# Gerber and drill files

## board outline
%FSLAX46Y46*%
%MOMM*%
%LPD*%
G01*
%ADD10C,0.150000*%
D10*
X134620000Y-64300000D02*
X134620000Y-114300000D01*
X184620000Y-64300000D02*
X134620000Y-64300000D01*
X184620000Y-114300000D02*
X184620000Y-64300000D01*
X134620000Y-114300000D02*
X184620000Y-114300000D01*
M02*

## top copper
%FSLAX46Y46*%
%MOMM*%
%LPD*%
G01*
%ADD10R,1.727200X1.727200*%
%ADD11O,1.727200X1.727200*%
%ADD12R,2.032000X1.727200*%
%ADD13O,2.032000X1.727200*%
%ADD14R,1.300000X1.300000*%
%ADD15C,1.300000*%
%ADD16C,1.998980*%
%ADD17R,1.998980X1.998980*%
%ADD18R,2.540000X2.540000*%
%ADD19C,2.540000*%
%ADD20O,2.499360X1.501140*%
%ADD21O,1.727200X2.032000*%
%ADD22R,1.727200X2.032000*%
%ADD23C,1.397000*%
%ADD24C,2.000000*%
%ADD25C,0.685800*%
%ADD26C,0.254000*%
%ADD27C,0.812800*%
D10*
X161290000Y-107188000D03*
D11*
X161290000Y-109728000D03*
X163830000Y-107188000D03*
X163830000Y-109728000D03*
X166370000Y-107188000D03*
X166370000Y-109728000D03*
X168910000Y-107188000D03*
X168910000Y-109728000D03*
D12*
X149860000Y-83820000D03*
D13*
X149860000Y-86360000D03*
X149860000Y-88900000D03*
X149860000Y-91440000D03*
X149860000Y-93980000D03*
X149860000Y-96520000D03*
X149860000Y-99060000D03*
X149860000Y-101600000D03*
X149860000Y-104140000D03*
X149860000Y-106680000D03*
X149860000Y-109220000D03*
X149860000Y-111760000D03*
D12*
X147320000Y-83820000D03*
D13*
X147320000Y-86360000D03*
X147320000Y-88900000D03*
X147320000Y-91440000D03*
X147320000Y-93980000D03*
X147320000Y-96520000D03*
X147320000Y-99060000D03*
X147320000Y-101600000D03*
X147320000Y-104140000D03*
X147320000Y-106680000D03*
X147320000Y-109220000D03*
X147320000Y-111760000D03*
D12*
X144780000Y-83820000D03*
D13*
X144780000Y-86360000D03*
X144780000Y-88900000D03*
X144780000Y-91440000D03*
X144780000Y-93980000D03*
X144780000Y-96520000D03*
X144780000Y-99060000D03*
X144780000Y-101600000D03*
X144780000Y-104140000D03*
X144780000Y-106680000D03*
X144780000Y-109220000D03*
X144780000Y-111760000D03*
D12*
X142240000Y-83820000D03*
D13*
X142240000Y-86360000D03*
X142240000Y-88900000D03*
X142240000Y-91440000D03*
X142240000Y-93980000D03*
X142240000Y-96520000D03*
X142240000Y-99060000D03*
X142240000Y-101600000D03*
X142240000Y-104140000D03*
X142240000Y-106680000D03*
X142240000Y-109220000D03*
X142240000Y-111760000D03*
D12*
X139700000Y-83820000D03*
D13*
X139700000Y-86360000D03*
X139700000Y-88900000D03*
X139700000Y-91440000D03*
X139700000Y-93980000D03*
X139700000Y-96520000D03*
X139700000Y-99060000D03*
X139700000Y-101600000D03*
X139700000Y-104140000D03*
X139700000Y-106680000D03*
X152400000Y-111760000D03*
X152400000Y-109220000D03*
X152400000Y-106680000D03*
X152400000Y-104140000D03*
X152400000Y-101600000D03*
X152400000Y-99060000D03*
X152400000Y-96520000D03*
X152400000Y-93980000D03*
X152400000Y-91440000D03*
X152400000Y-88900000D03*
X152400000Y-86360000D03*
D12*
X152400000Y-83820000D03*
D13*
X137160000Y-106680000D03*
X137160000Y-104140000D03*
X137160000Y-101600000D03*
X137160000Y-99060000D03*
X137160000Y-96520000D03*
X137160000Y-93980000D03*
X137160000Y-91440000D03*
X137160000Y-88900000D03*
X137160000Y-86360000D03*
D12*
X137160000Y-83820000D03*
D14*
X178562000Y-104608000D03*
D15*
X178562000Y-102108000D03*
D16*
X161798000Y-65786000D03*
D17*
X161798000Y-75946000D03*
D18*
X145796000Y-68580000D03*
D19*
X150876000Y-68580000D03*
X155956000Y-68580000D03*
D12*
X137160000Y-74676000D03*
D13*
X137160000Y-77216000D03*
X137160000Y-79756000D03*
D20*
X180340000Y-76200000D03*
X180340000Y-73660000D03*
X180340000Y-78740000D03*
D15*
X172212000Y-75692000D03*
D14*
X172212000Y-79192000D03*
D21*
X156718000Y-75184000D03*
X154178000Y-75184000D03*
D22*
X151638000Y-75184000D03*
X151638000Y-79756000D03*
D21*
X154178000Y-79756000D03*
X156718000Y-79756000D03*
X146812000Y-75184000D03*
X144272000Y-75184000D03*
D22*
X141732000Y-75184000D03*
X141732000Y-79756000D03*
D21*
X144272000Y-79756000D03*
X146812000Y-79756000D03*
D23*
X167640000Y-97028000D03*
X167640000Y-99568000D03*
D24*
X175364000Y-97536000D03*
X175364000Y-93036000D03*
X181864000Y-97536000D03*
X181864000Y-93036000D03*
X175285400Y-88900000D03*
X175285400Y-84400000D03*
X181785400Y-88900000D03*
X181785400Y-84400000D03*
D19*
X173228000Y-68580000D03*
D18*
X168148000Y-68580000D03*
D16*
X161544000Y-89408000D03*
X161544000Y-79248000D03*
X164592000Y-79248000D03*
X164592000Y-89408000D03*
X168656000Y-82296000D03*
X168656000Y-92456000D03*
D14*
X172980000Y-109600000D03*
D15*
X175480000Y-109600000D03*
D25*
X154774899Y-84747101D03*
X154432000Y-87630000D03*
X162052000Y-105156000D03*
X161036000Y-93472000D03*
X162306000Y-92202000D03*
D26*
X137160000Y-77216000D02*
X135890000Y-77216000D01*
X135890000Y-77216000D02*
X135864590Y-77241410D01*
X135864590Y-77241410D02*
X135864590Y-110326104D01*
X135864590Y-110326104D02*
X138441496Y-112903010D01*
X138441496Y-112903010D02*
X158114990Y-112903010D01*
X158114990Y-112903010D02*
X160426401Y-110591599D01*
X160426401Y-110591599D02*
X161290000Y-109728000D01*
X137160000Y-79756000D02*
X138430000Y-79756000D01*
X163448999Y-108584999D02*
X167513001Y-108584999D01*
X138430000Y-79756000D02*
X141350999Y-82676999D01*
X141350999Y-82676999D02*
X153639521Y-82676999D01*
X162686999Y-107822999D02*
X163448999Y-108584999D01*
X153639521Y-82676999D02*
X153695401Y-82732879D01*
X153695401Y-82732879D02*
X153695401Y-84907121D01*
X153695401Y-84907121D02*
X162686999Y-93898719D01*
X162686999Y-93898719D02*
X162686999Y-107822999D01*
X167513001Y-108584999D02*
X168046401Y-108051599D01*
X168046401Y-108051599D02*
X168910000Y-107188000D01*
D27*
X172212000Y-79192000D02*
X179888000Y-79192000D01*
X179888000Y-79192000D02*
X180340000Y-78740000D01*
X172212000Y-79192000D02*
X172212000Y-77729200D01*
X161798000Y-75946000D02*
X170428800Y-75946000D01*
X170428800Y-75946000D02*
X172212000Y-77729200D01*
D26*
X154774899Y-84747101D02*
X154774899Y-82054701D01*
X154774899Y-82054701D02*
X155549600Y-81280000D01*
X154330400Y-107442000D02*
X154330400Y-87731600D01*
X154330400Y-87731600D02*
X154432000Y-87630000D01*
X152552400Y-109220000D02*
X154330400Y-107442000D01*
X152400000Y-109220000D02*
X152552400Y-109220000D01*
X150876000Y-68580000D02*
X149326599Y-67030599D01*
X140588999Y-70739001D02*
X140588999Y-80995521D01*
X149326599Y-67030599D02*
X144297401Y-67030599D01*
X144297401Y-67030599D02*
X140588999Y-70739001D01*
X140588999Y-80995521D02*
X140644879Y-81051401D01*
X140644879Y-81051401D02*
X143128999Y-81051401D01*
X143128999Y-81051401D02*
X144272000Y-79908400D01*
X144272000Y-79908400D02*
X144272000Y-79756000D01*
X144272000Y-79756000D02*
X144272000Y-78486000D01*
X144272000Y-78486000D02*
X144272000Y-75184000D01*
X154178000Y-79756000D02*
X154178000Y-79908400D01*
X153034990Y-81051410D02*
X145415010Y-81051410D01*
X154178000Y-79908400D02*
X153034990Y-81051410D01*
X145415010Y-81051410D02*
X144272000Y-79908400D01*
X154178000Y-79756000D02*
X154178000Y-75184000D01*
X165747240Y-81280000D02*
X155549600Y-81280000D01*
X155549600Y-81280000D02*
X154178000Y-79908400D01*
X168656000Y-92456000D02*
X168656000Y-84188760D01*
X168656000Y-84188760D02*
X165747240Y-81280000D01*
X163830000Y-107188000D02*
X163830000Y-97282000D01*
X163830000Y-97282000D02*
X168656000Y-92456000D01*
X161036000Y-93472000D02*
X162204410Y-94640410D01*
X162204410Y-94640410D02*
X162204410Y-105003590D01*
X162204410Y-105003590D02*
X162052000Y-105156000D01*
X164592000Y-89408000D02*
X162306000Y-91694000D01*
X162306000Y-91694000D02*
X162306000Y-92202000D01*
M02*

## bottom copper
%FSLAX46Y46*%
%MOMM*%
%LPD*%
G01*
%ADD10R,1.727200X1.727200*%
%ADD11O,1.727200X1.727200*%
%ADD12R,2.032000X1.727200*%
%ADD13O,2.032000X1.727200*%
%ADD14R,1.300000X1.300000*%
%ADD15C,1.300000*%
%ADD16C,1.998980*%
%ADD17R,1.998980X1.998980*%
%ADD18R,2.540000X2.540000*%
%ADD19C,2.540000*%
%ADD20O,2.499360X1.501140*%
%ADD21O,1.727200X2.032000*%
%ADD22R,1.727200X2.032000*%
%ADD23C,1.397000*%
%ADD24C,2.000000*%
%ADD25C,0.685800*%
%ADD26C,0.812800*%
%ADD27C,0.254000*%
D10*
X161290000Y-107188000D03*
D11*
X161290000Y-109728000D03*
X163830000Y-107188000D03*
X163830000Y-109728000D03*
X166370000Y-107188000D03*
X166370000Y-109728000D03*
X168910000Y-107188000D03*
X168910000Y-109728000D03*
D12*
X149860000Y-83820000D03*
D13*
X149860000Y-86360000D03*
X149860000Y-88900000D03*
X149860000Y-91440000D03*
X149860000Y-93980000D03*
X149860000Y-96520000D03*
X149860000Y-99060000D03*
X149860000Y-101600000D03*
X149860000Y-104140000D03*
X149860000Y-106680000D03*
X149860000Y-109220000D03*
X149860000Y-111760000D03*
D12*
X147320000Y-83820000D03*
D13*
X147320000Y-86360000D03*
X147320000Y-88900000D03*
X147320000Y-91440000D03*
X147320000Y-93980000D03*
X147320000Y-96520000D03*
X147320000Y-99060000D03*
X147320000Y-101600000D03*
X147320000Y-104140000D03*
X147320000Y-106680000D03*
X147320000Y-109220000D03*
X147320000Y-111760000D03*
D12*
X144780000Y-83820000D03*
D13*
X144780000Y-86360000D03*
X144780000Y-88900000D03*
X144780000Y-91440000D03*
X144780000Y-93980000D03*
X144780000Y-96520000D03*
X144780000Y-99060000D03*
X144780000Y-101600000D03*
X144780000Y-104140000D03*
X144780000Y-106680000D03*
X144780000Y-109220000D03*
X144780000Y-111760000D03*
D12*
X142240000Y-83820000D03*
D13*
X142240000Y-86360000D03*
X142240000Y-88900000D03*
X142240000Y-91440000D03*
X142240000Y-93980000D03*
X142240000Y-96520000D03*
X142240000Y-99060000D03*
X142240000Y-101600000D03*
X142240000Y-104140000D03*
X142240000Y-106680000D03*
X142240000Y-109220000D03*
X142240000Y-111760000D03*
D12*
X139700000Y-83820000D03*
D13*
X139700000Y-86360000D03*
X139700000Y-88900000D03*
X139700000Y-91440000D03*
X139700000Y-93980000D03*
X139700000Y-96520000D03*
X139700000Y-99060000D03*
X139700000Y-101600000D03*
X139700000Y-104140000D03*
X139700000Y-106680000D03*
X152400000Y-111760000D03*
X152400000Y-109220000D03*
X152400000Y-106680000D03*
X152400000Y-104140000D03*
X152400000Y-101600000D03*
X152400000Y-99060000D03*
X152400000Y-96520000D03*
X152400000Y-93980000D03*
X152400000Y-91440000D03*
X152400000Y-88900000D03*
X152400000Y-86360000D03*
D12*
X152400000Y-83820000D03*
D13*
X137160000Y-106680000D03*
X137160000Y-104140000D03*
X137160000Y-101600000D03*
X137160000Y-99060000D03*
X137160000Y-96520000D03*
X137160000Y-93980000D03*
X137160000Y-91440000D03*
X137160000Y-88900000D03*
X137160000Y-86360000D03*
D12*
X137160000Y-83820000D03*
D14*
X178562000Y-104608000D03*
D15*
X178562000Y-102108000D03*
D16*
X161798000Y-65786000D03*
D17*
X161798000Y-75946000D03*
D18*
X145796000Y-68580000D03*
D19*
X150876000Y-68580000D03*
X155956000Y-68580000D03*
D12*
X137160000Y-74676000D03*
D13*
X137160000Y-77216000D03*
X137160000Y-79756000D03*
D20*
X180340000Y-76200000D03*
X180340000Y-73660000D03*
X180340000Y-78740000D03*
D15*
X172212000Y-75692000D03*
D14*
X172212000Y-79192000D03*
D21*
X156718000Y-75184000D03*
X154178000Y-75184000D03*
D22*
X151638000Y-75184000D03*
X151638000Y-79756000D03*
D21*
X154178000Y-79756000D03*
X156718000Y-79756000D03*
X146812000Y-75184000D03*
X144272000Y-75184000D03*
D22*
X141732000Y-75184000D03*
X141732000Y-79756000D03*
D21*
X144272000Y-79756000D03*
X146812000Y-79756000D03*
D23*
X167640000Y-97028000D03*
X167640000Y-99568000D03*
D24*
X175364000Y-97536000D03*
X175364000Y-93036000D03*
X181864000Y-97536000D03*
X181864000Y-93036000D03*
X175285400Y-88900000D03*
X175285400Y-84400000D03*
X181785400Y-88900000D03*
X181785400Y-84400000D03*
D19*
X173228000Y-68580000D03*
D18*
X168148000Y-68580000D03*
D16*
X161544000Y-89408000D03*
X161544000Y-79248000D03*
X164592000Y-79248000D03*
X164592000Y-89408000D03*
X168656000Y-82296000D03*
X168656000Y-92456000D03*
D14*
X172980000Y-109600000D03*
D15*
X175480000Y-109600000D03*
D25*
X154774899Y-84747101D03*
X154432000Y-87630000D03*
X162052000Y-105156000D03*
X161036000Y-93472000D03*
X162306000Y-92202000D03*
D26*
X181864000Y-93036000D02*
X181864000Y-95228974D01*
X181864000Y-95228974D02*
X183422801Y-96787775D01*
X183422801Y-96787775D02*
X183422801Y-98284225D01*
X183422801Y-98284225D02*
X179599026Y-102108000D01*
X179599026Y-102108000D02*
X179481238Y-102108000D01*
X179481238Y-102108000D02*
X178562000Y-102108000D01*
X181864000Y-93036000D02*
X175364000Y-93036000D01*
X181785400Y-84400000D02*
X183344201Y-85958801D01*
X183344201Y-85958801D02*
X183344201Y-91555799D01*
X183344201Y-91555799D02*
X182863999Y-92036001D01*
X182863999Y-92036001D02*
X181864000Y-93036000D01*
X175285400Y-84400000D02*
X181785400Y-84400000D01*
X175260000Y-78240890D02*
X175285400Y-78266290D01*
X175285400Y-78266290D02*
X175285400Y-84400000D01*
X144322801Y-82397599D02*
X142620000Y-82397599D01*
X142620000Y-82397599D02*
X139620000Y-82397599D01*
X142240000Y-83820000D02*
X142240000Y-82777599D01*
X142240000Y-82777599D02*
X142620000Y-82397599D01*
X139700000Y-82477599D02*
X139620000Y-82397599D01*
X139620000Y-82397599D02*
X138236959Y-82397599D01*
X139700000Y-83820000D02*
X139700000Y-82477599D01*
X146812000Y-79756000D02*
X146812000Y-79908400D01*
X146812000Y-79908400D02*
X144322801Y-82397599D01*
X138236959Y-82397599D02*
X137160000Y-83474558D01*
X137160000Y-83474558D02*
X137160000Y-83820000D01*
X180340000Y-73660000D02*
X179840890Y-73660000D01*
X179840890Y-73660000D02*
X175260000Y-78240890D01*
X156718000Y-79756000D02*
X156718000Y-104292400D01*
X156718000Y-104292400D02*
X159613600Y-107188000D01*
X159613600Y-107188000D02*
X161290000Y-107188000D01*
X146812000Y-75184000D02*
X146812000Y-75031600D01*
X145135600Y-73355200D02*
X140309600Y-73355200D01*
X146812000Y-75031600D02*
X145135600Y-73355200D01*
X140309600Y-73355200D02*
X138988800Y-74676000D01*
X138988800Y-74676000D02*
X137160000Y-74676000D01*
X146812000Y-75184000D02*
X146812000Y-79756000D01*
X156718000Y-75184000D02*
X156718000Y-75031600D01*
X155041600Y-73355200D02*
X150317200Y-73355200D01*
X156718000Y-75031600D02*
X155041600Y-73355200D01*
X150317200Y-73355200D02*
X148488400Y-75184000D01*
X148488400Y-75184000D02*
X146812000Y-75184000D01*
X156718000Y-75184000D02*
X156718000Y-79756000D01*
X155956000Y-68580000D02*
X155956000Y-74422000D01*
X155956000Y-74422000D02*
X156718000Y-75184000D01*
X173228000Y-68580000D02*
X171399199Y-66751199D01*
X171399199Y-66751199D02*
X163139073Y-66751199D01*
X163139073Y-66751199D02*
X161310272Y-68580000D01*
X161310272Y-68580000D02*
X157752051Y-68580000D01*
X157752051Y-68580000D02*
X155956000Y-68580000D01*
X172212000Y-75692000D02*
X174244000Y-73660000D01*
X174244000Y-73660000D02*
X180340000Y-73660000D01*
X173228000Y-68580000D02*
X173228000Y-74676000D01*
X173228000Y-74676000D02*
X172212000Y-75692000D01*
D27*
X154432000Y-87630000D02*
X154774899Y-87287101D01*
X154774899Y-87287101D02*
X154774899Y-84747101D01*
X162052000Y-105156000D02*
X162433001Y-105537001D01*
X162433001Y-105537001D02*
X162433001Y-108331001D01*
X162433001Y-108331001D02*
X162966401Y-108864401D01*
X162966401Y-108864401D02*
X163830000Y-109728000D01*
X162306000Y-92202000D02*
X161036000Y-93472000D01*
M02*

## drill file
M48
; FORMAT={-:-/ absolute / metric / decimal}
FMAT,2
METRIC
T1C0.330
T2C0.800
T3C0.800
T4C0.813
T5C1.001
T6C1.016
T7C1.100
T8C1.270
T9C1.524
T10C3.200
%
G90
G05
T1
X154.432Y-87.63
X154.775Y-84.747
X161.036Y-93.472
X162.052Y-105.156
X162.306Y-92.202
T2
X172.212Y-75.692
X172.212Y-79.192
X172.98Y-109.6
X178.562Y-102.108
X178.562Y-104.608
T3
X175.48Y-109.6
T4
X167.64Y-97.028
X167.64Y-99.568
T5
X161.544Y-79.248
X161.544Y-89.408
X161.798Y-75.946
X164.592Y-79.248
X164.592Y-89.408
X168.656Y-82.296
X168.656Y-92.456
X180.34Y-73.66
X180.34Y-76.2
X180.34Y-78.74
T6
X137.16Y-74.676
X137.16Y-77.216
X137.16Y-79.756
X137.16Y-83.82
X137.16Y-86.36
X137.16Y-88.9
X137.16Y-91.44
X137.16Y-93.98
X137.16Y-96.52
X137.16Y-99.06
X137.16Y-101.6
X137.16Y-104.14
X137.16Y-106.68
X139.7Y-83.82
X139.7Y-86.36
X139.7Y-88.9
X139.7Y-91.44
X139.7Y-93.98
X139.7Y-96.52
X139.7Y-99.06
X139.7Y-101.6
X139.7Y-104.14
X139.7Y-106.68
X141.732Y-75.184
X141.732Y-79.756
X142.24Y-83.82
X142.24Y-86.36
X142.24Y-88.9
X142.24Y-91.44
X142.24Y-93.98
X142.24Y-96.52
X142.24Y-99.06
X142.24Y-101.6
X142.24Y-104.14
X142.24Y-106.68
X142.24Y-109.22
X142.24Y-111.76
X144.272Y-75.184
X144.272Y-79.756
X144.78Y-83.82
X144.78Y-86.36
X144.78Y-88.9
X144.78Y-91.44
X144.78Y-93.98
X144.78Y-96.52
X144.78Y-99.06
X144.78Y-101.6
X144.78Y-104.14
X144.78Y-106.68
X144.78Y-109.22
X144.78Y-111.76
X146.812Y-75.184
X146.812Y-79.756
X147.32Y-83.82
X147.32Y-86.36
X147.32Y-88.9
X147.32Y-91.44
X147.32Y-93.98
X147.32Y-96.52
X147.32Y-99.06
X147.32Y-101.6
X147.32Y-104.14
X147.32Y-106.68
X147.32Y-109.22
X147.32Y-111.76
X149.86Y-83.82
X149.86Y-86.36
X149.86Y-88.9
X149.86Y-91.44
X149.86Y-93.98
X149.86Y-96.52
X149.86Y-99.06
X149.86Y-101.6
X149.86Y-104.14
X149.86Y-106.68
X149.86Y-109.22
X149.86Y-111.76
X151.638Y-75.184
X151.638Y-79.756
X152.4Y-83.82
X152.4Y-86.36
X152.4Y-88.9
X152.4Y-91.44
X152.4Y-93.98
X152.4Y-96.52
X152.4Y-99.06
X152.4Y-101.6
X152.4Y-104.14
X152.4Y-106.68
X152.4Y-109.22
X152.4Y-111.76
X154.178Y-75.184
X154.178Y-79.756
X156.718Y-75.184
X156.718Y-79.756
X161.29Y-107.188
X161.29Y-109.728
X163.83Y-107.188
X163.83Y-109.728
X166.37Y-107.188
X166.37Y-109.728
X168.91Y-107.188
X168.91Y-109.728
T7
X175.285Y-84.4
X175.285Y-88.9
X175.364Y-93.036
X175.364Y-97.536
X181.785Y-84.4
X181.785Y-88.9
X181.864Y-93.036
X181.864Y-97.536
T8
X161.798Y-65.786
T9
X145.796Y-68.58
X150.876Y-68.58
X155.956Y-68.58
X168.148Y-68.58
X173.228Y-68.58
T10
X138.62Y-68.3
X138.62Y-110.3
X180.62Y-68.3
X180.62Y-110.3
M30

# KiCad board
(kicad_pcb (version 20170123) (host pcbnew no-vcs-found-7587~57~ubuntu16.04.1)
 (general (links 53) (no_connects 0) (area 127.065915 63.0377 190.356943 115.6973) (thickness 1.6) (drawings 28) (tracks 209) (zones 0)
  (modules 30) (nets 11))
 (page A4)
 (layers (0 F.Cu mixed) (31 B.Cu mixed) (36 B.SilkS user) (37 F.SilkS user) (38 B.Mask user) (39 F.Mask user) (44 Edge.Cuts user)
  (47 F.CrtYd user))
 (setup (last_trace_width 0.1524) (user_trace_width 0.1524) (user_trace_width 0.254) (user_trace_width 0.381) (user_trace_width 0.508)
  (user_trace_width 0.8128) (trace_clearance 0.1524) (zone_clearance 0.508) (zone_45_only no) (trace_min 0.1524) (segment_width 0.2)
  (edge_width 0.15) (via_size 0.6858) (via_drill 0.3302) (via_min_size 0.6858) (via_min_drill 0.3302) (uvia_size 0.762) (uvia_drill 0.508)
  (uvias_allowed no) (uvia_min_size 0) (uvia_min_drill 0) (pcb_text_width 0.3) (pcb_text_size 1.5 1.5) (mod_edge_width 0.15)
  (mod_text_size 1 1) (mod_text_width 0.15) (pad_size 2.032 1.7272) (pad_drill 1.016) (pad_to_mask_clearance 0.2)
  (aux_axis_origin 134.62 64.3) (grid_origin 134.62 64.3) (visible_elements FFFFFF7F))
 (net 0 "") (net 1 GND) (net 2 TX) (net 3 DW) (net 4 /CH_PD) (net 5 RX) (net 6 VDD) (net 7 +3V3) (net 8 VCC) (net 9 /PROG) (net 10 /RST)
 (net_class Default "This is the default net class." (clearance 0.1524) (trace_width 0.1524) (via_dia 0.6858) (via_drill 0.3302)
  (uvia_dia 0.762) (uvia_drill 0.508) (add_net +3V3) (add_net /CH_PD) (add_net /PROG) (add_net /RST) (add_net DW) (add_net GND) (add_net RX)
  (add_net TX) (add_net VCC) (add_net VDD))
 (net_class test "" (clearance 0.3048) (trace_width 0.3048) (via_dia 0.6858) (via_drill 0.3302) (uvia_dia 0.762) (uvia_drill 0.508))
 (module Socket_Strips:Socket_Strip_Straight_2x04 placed (layer F.Cu) (at 161.29 107.188)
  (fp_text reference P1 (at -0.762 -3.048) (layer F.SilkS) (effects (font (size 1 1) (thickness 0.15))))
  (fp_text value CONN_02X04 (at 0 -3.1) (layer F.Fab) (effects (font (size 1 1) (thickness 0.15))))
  (pad 1 thru_hole rect (at 0 0) (size 1.7272 1.7272) (drill 1.016) (layers *.Cu *.Mask) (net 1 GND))
  (pad 2 thru_hole oval (at 0 2.54) (size 1.7272 1.7272) (drill 1.016) (layers *.Cu *.Mask) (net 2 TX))
  (pad 3 thru_hole oval (at 2.54 0) (size 1.7272 1.7272) (drill 1.016) (layers *.Cu *.Mask) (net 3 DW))
  (pad 4 thru_hole oval (at 2.54 2.54) (size 1.7272 1.7272) (drill 1.016) (layers *.Cu *.Mask) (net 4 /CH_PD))
  (pad 5 thru_hole oval (at 5.08 0) (size 1.7272 1.7272) (drill 1.016) (layers *.Cu *.Mask))
  (pad 6 thru_hole oval (at 5.08 2.54) (size 1.7272 1.7272) (drill 1.016) (layers *.Cu *.Mask))
  (pad 7 thru_hole oval (at 7.62 0) (size 1.7272 1.7272) (drill 1.016) (layers *.Cu *.Mask) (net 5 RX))
  (pad 8 thru_hole oval (at 7.62 2.54) (size 1.7272 1.7272) (drill 1.016) (layers *.Cu *.Mask)))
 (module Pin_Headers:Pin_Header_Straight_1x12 (layer F.Cu) (at 149.86 83.82)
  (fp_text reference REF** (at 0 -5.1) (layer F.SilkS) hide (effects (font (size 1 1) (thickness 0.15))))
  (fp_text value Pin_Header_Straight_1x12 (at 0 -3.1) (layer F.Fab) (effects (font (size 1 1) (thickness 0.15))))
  (pad 1 thru_hole rect (at 0 0) (size 2.032 1.7272) (drill 1.016) (layers *.Cu *.Mask))
  (pad 2 thru_hole oval (at 0 2.54) (size 2.032 1.7272) (drill 1.016) (layers *.Cu *.Mask))
  (pad 3 thru_hole oval (at 0 5.08) (size 2.032 1.7272) (drill 1.016) (layers *.Cu *.Mask))
  (pad 4 thru_hole oval (at 0 7.62) (size 2.032 1.7272) (drill 1.016) (layers *.Cu *.Mask))
  (pad 5 thru_hole oval (at 0 10.16) (size 2.032 1.7272) (drill 1.016) (layers *.Cu *.Mask))
  (pad 6 thru_hole oval (at 0 12.7) (size 2.032 1.7272) (drill 1.016) (layers *.Cu *.Mask))
  (pad 7 thru_hole oval (at 0 15.24) (size 2.032 1.7272) (drill 1.016) (layers *.Cu *.Mask))
  (pad 8 thru_hole oval (at 0 17.78) (size 2.032 1.7272) (drill 1.016) (layers *.Cu *.Mask))
  (pad 9 thru_hole oval (at 0 20.32) (size 2.032 1.7272) (drill 1.016) (layers *.Cu *.Mask))
  (pad 10 thru_hole oval (at 0 22.86) (size 2.032 1.7272) (drill 1.016) (layers *.Cu *.Mask))
  (pad 11 thru_hole oval (at 0 25.4) (size 2.032 1.7272) (drill 1.016) (layers *.Cu *.Mask))
  (pad 12 thru_hole oval (at 0 27.94) (size 2.032 1.7272) (drill 1.016) (layers *.Cu *.Mask)))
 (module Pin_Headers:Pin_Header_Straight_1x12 (layer F.Cu) (at 147.32 83.82)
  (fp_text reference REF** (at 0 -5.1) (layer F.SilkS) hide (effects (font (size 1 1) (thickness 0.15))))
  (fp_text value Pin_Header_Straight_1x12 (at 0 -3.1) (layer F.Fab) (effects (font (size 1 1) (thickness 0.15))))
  (pad 1 thru_hole rect (at 0 0) (size 2.032 1.7272) (drill 1.016) (layers *.Cu *.Mask))
  (pad 2 thru_hole oval (at 0 2.54) (size 2.032 1.7272) (drill 1.016) (layers *.Cu *.Mask))
  (pad 3 thru_hole oval (at 0 5.08) (size 2.032 1.7272) (drill 1.016) (layers *.Cu *.Mask))
  (pad 4 thru_hole oval (at 0 7.62) (size 2.032 1.7272) (drill 1.016) (layers *.Cu *.Mask))
  (pad 5 thru_hole oval (at 0 10.16) (size 2.032 1.7272) (drill 1.016) (layers *.Cu *.Mask))
  (pad 6 thru_hole oval (at 0 12.7) (size 2.032 1.7272) (drill 1.016) (layers *.Cu *.Mask))
  (pad 7 thru_hole oval (at 0 15.24) (size 2.032 1.7272) (drill 1.016) (layers *.Cu *.Mask))
  (pad 8 thru_hole oval (at 0 17.78) (size 2.032 1.7272) (drill 1.016) (layers *.Cu *.Mask))
  (pad 9 thru_hole oval (at 0 20.32) (size 2.032 1.7272) (drill 1.016) (layers *.Cu *.Mask))
  (pad 10 thru_hole oval (at 0 22.86) (size 2.032 1.7272) (drill 1.016) (layers *.Cu *.Mask))
  (pad 11 thru_hole oval (at 0 25.4) (size 2.032 1.7272) (drill 1.016) (layers *.Cu *.Mask))
  (pad 12 thru_hole oval (at 0 27.94) (size 2.032 1.7272) (drill 1.016) (layers *.Cu *.Mask)))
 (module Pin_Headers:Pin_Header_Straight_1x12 (layer F.Cu) (at 144.78 83.82)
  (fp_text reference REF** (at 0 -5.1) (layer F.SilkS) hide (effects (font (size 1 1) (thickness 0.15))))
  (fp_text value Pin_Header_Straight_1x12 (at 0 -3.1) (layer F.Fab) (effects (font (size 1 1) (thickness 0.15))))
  (pad 1 thru_hole rect (at 0 0) (size 2.032 1.7272) (drill 1.016) (layers *.Cu *.Mask))
  (pad 2 thru_hole oval (at 0 2.54) (size 2.032 1.7272) (drill 1.016) (layers *.Cu *.Mask))
  (pad 3 thru_hole oval (at 0 5.08) (size 2.032 1.7272) (drill 1.016) (layers *.Cu *.Mask))
  (pad 4 thru_hole oval (at 0 7.62) (size 2.032 1.7272) (drill 1.016) (layers *.Cu *.Mask))
  (pad 5 thru_hole oval (at 0 10.16) (size 2.032 1.7272) (drill 1.016) (layers *.Cu *.Mask))
  (pad 6 thru_hole oval (at 0 12.7) (size 2.032 1.7272) (drill 1.016) (layers *.Cu *.Mask))
  (pad 7 thru_hole oval (at 0 15.24) (size 2.032 1.7272) (drill 1.016) (layers *.Cu *.Mask))
  (pad 8 thru_hole oval (at 0 17.78) (size 2.032 1.7272) (drill 1.016) (layers *.Cu *.Mask))
  (pad 9 thru_hole oval (at 0 20.32) (size 2.032 1.7272) (drill 1.016) (layers *.Cu *.Mask))
  (pad 10 thru_hole oval (at 0 22.86) (size 2.032 1.7272) (drill 1.016) (layers *.Cu *.Mask))
  (pad 11 thru_hole oval (at 0 25.4) (size 2.032 1.7272) (drill 1.016) (layers *.Cu *.Mask))
  (pad 12 thru_hole oval (at 0 27.94) (size 2.032 1.7272) (drill 1.016) (layers *.Cu *.Mask)))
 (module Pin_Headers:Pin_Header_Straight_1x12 (layer F.Cu) (at 142.24 83.82)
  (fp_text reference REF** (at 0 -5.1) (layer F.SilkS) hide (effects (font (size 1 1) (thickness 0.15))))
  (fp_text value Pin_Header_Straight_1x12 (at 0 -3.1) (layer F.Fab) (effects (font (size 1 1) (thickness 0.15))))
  (pad 1 thru_hole rect (at 0 0) (size 2.032 1.7272) (drill 1.016) (layers *.Cu *.Mask) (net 1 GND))
  (pad 2 thru_hole oval (at 0 2.54) (size 2.032 1.7272) (drill 1.016) (layers *.Cu *.Mask))
  (pad 3 thru_hole oval (at 0 5.08) (size 2.032 1.7272) (drill 1.016) (layers *.Cu *.Mask))
  (pad 4 thru_hole oval (at 0 7.62) (size 2.032 1.7272) (drill 1.016) (layers *.Cu *.Mask))
  (pad 5 thru_hole oval (at 0 10.16) (size 2.032 1.7272) (drill 1.016) (layers *.Cu *.Mask))
  (pad 6 thru_hole oval (at 0 12.7) (size 2.032 1.7272) (drill 1.016) (layers *.Cu *.Mask))
  (pad 7 thru_hole oval (at 0 15.24) (size 2.032 1.7272) (drill 1.016) (layers *.Cu *.Mask))
  (pad 8 thru_hole oval (at 0 17.78) (size 2.032 1.7272) (drill 1.016) (layers *.Cu *.Mask))
  (pad 9 thru_hole oval (at 0 20.32) (size 2.032 1.7272) (drill 1.016) (layers *.Cu *.Mask))
  (pad 10 thru_hole oval (at 0 22.86) (size 2.032 1.7272) (drill 1.016) (layers *.Cu *.Mask))
  (pad 11 thru_hole oval (at 0 25.4) (size 2.032 1.7272) (drill 1.016) (layers *.Cu *.Mask))
  (pad 12 thru_hole oval (at 0 27.94) (size 2.032 1.7272) (drill 1.016) (layers *.Cu *.Mask)))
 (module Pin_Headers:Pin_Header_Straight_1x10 (layer F.Cu) (at 139.7 83.82)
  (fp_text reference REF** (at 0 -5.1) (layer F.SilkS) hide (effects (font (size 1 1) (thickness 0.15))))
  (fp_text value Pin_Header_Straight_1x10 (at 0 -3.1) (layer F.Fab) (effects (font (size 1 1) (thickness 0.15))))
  (pad 1 thru_hole rect (at 0 0) (size 2.032 1.7272) (drill 1.016) (layers *.Cu *.Mask) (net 1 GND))
  (pad 2 thru_hole oval (at 0 2.54) (size 2.032 1.7272) (drill 1.016) (layers *.Cu *.Mask))
  (pad 3 thru_hole oval (at 0 5.08) (size 2.032 1.7272) (drill 1.016) (layers *.Cu *.Mask))
  (pad 4 thru_hole oval (at 0 7.62) (size 2.032 1.7272) (drill 1.016) (layers *.Cu *.Mask))
  (pad 5 thru_hole oval (at 0 10.16) (size 2.032 1.7272) (drill 1.016) (layers *.Cu *.Mask))
  (pad 6 thru_hole oval (at 0 12.7) (size 2.032 1.7272) (drill 1.016) (layers *.Cu *.Mask))
  (pad 7 thru_hole oval (at 0 15.24) (size 2.032 1.7272) (drill 1.016) (layers *.Cu *.Mask))
  (pad 8 thru_hole oval (at 0 17.78) (size 2.032 1.7272) (drill 1.016) (layers *.Cu *.Mask))
  (pad 9 thru_hole oval (at 0 20.32) (size 2.032 1.7272) (drill 1.016) (layers *.Cu *.Mask))
  (pad 10 thru_hole oval (at 0 22.86) (size 2.032 1.7272) (drill 1.016) (layers *.Cu *.Mask)))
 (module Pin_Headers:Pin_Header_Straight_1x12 (layer F.Cu) (at 152.4 83.82)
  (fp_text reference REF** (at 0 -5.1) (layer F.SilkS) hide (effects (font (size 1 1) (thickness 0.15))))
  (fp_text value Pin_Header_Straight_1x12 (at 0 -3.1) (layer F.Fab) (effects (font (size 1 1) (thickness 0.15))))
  (pad 12 thru_hole oval (at 0 27.94) (size 2.032 1.7272) (drill 1.016) (layers *.Cu *.Mask))
  (pad 11 thru_hole oval (at 0 25.4) (size 2.032 1.7272) (drill 1.016) (layers *.Cu *.Mask) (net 3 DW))
  (pad 10 thru_hole oval (at 0 22.86) (size 2.032 1.7272) (drill 1.016) (layers *.Cu *.Mask))
  (pad 9 thru_hole oval (at 0 20.32) (size 2.032 1.7272) (drill 1.016) (layers *.Cu *.Mask))
  (pad 8 thru_hole oval (at 0 17.78) (size 2.032 1.7272) (drill 1.016) (layers *.Cu *.Mask))
  (pad 7 thru_hole oval (at 0 15.24) (size 2.032 1.7272) (drill 1.016) (layers *.Cu *.Mask))
  (pad 6 thru_hole oval (at 0 12.7) (size 2.032 1.7272) (drill 1.016) (layers *.Cu *.Mask))
  (pad 5 thru_hole oval (at 0 10.16) (size 2.032 1.7272) (drill 1.016) (layers *.Cu *.Mask))
  (pad 4 thru_hole oval (at 0 7.62) (size 2.032 1.7272) (drill 1.016) (layers *.Cu *.Mask))
  (pad 3 thru_hole oval (at 0 5.08) (size 2.032 1.7272) (drill 1.016) (layers *.Cu *.Mask))
  (pad 2 thru_hole oval (at 0 2.54) (size 2.032 1.7272) (drill 1.016) (layers *.Cu *.Mask))
  (pad 1 thru_hole rect (at 0 0) (size 2.032 1.7272) (drill 1.016) (layers *.Cu *.Mask)))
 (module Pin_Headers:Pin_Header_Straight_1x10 (layer F.Cu) (at 137.16 83.82)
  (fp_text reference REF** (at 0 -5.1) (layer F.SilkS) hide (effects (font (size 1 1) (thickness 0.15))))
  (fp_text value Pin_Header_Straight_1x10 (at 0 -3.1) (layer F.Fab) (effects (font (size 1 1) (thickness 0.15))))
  (pad 10 thru_hole oval (at 0 22.86) (size 2.032 1.7272) (drill 1.016) (layers *.Cu *.Mask))
  (pad 9 thru_hole oval (at 0 20.32) (size 2.032 1.7272) (drill 1.016) (layers *.Cu *.Mask))
  (pad 8 thru_hole oval (at 0 17.78) (size 2.032 1.7272) (drill 1.016) (layers *.Cu *.Mask))
  (pad 7 thru_hole oval (at 0 15.24) (size 2.032 1.7272) (drill 1.016) (layers *.Cu *.Mask))
  (pad 6 thru_hole oval (at 0 12.7) (size 2.032 1.7272) (drill 1.016) (layers *.Cu *.Mask))
  (pad 5 thru_hole oval (at 0 10.16) (size 2.032 1.7272) (drill 1.016) (layers *.Cu *.Mask))
  (pad 4 thru_hole oval (at 0 7.62) (size 2.032 1.7272) (drill 1.016) (layers *.Cu *.Mask))
  (pad 3 thru_hole oval (at 0 5.08) (size 2.032 1.7272) (drill 1.016) (layers *.Cu *.Mask))
  (pad 2 thru_hole oval (at 0 2.54) (size 2.032 1.7272) (drill 1.016) (layers *.Cu *.Mask))
  (pad 1 thru_hole rect (at 0 0) (size 2.032 1.7272) (drill 1.016) (layers *.Cu *.Mask) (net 1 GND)))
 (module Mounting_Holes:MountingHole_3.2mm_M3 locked (layer F.Cu) (at 180.62 68.3)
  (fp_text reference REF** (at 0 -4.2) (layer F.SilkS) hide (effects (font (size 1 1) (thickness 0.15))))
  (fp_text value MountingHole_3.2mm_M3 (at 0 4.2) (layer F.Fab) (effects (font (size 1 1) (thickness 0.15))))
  (pad 1 np_thru_hole circle (at 0 0) (size 3.2 3.2) (drill 3.2) (layers *.Cu *.Mask)))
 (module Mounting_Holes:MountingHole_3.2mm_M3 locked (layer F.Cu) (at 138.62 68.3)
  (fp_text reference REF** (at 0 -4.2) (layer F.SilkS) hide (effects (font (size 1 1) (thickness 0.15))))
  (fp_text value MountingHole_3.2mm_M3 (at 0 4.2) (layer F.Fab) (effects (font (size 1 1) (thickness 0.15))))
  (pad 1 np_thru_hole circle (at 0 0) (size 3.2 3.2) (drill 3.2) (layers *.Cu *.Mask)))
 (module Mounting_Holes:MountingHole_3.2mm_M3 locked (layer F.Cu) (at 138.62 110.3)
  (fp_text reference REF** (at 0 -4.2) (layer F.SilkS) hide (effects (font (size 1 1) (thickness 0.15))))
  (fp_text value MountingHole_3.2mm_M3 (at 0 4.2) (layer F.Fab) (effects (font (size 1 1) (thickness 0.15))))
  (pad 1 np_thru_hole circle (at 0 0) (size 3.2 3.2) (drill 3.2) (layers *.Cu *.Mask)))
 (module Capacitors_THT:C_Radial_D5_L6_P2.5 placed (layer F.Cu) (at 178.562 104.608 90)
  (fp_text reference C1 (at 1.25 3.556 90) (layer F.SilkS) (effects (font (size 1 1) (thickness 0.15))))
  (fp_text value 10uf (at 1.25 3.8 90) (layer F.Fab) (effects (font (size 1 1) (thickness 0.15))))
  (pad 1 thru_hole rect (at 0 0 90) (size 1.3 1.3) (drill 0.8) (layers *.Cu *.Mask))
  (pad 2 thru_hole circle (at 2.5 0 90) (size 1.3 1.3) (drill 0.8) (layers *.Cu *.Mask) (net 1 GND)))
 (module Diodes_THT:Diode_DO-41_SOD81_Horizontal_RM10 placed (layer F.Cu) (at 161.80054 75.946 90)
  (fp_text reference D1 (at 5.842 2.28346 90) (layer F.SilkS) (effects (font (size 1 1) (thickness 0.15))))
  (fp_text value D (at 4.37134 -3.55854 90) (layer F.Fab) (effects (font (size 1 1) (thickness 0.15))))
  (pad 2 thru_hole circle (at 10.16 -0.00254 270) (size 1.99898 1.99898) (drill 1.27) (layers *.Cu *.Mask))
  (pad 1 thru_hole rect (at 0 -0.00254 270) (size 1.99898 1.99898) (drill 1.00076) (layers *.Cu *.Mask) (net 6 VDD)))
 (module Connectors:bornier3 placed (layer F.Cu) (at 150.876 68.58)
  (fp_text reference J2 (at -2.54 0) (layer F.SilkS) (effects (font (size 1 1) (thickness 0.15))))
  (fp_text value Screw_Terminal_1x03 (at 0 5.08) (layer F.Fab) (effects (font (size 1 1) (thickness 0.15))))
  (pad 1 thru_hole rect (at -5.08 0) (size 2.54 2.54) (drill 1.524) (layers *.Cu *.Mask))
  (pad 2 thru_hole circle (at 0 0) (size 2.54 2.54) (drill 1.524) (layers *.Cu *.Mask) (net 3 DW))
  (pad 3 thru_hole circle (at 5.08 0) (size 2.54 2.54) (drill 1.524) (layers *.Cu *.Mask) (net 1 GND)))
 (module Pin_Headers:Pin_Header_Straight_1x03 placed (layer F.Cu) (at 137.16 74.676)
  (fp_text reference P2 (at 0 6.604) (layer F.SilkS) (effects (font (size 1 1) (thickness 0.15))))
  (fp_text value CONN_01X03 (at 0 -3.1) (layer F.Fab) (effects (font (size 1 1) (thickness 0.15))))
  (pad 1 thru_hole rect (at 0 0) (size 2.032 1.7272) (drill 1.016) (layers *.Cu *.Mask) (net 1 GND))
  (pad 2 thru_hole oval (at 0 2.54) (size 2.032 1.7272) (drill 1.016) (layers *.Cu *.Mask) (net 2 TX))
  (pad 3 thru_hole oval (at 0 5.08) (size 2.032 1.7272) (drill 1.016) (layers *.Cu *.Mask) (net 5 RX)))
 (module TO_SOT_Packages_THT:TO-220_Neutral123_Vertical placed (layer F.Cu) (at 180.34 76.2 270)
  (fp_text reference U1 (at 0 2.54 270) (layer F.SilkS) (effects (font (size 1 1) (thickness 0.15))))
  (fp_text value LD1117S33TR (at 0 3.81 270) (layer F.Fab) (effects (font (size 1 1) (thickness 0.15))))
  (pad 2 thru_hole oval (at 0 0) (size 2.49936 1.50114) (drill 1.00076) (layers *.Cu *.Mask))
  (pad 1 thru_hole oval (at -2.54 0) (size 2.49936 1.50114) (drill 1.00076) (layers *.Cu *.Mask) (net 1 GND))
  (pad 3 thru_hole oval (at 2.54 0) (size 2.49936 1.50114) (drill 1.00076) (layers *.Cu *.Mask) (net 6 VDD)))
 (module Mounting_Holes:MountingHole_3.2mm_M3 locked (layer F.Cu) (at 180.62 110.3)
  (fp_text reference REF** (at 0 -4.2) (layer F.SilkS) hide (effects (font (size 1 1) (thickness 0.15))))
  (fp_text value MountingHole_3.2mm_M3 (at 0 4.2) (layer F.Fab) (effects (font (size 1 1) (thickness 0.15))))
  (pad 1 np_thru_hole circle (at 0 0) (size 3.2 3.2) (drill 3.2) (layers *.Cu *.Mask)))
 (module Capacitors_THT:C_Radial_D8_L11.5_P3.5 (layer F.Cu) (at 172.212 79.192 90)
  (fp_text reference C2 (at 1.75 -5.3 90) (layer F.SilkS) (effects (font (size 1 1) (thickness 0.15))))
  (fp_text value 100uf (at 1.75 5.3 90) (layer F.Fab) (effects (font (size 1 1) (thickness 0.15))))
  (pad 2 thru_hole circle (at 3.5 0 90) (size 1.3 1.3) (drill 0.8) (layers *.Cu *.Mask) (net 1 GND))
  (pad 1 thru_hole rect (at 0 0 90) (size 1.3 1.3) (drill 0.8) (layers *.Cu *.Mask) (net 6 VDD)))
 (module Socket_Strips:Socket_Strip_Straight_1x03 (layer F.Cu) (at 151.638 75.184)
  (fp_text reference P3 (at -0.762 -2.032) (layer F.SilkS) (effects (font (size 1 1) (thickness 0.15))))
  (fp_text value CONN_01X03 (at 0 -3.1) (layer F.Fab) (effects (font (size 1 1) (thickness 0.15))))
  (pad 3 thru_hole oval (at 5.08 0) (size 1.7272 2.032) (drill 1.016) (layers *.Cu *.Mask) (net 1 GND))
  (pad 2 thru_hole oval (at 2.54 0) (size 1.7272 2.032) (drill 1.016) (layers *.Cu *.Mask) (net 3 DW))
  (pad 1 thru_hole rect (at 0 0) (size 1.7272 2.032) (drill 1.016) (layers *.Cu *.Mask)))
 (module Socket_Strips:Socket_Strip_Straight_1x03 (layer F.Cu) (at 151.638 79.756)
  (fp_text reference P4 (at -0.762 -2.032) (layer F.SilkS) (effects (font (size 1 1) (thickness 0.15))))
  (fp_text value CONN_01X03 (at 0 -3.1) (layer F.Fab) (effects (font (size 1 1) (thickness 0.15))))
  (pad 1 thru_hole rect (at 0 0) (size 1.7272 2.032) (drill 1.016) (layers *.Cu *.Mask))
  (pad 2 thru_hole oval (at 2.54 0) (size 1.7272 2.032) (drill 1.016) (layers *.Cu *.Mask) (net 3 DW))
  (pad 3 thru_hole oval (at 5.08 0) (size 1.7272 2.032) (drill 1.016) (layers *.Cu *.Mask) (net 1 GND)))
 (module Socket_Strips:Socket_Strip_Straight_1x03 (layer F.Cu) (at 141.732 75.184)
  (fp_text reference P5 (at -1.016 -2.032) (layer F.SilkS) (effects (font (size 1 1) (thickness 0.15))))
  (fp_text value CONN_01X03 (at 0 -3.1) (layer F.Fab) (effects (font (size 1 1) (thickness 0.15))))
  (pad 3 thru_hole oval (at 5.08 0) (size 1.7272 2.032) (drill 1.016) (layers *.Cu *.Mask) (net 1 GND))
  (pad 2 thru_hole oval (at 2.54 0) (size 1.7272 2.032) (drill 1.016) (layers *.Cu *.Mask) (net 3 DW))
  (pad 1 thru_hole rect (at 0 0) (size 1.7272 2.032) (drill 1.016) (layers *.Cu *.Mask)))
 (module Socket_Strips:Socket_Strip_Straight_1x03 (layer F.Cu) (at 141.732 79.756)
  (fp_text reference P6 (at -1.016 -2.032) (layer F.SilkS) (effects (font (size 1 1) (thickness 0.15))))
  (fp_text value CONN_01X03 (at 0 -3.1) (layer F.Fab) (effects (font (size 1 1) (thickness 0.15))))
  (pad 1 thru_hole rect (at 0 0) (size 1.7272 2.032) (drill 1.016) (layers *.Cu *.Mask))
  (pad 2 thru_hole oval (at 2.54 0) (size 1.7272 2.032) (drill 1.016) (layers *.Cu *.Mask) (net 3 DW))
  (pad 3 thru_hole oval (at 5.08 0) (size 1.7272 2.032) (drill 1.016) (layers *.Cu *.Mask) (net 1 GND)))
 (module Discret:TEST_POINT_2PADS (layer F.Cu) (at 167.64 98.298 270)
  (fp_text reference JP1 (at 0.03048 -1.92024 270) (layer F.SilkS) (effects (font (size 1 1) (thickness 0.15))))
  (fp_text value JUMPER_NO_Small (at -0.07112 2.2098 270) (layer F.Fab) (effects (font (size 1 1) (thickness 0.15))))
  (pad 1 thru_hole circle (at -1.27 0 270) (size 1.397 1.397) (drill 0.8128) (layers *.Cu *.Mask F.SilkS))
  (pad 2 thru_hole circle (at 1.27 0 270) (size 1.397 1.397) (drill 0.8128) (layers *.Cu *.Mask F.SilkS)))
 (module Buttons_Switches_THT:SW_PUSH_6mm (layer F.Cu) (at 181.864 97.536 180)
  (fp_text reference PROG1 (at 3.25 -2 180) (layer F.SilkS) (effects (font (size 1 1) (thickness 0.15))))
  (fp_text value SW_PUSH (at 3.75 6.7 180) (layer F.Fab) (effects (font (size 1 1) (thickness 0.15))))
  (pad 1 thru_hole circle (at 6.5 0 270) (size 2 2) (drill 1.1) (layers *.Cu *.Mask))
  (pad 2 thru_hole circle (at 6.5 4.5 270) (size 2 2) (drill 1.1) (layers *.Cu *.Mask) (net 1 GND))
  (pad 1 thru_hole circle (at 0 0 270) (size 2 2) (drill 1.1) (layers *.Cu *.Mask))
  (pad 2 thru_hole circle (at 0 4.5 270) (size 2 2) (drill 1.1) (layers *.Cu *.Mask) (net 1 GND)))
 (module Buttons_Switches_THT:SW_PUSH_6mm (layer F.Cu) (at 175.2854 84.4)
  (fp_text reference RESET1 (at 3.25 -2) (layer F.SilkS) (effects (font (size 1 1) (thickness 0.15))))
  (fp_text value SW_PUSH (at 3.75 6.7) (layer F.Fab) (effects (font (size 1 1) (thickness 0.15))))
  (pad 2 thru_hole circle (at 0 4.5 90) (size 2 2) (drill 1.1) (layers *.Cu *.Mask))
  (pad 1 thru_hole circle (at 0 0 90) (size 2 2) (drill 1.1) (layers *.Cu *.Mask) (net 1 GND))
  (pad 2 thru_hole circle (at 6.5 4.5 90) (size 2 2) (drill 1.1) (layers *.Cu *.Mask))
  (pad 1 thru_hole circle (at 6.5 0 90) (size 2 2) (drill 1.1) (layers *.Cu *.Mask) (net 1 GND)))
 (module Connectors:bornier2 (layer F.Cu) (at 170.688 68.58)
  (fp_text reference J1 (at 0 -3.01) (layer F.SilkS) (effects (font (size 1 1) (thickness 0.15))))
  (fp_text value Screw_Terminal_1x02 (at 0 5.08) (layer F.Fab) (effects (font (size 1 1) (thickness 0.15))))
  (pad 2 thru_hole circle (at 2.54 0) (size 2.54 2.54) (drill 1.524) (layers *.Cu *.Mask) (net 1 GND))
  (pad 1 thru_hole rect (at -2.54 0) (size 2.54 2.54) (drill 1.524) (layers *.Cu *.Mask)))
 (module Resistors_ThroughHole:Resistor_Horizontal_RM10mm (layer F.Cu) (at 161.544 89.408 90)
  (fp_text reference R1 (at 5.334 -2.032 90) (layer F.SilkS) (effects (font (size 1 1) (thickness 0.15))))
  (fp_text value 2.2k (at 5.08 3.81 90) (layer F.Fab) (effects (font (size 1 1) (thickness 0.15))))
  (pad 1 thru_hole circle (at 0 0 90) (size 1.99898 1.99898) (drill 1.00076) (layers *.Cu *.SilkS *.Mask))
  (pad 2 thru_hole circle (at 10.16 0 90) (size 1.99898 1.99898) (drill 1.00076) (layers *.Cu *.SilkS *.Mask)))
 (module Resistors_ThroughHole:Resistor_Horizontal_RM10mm (layer F.Cu) (at 164.592 89.408 90)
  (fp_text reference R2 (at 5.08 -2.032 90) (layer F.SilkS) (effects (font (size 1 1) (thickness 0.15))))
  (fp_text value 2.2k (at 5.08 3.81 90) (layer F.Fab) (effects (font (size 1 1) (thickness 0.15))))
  (pad 2 thru_hole circle (at 10.16 0 90) (size 1.99898 1.99898) (drill 1.00076) (layers *.Cu *.SilkS *.Mask))
  (pad 1 thru_hole circle (at 0 0 90) (size 1.99898 1.99898) (drill 1.00076) (layers *.Cu *.SilkS *.Mask) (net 4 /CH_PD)))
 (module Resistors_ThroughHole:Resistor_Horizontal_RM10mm (layer F.Cu) (at 168.656 82.296 270)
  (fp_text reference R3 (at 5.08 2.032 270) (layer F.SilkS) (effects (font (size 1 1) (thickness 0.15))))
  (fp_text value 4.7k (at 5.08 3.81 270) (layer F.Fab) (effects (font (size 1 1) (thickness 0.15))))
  (pad 1 thru_hole circle (at 0 0 270) (size 1.99898 1.99898) (drill 1.00076) (layers *.Cu *.SilkS *.Mask))
  (pad 2 thru_hole circle (at 10.16 0 270) (size 1.99898 1.99898) (drill 1.00076) (layers *.Cu *.SilkS *.Mask) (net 3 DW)))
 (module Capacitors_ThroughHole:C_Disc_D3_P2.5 (layer F.Cu) (at 172.98 109.6)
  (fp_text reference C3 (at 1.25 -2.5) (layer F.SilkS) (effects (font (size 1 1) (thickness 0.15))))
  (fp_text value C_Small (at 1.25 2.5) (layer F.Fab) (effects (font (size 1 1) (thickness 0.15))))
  (pad 1 thru_hole rect (at 0 0) (size 1.3 1.3) (drill 0.8) (layers *.Cu *.Mask F.SilkS))
  (pad 2 thru_hole circle (at 2.5 0) (size 1.3 1.3) (drill 0.8001) (layers *.Cu *.Mask F.SilkS)))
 (gr_line (start 134.62 64.3) (end 134.62 114.3) (angle 90) (layer Edge.Cuts) (width 0.15))
 (gr_line (start 184.62 64.3) (end 134.62 64.3) (angle 90) (layer Edge.Cuts) (width 0.15))
 (gr_line (start 184.62 114.3) (end 184.62 64.3) (angle 90) (layer Edge.Cuts) (width 0.15))
 (gr_line (start 134.62 114.3) (end 184.62 114.3) (angle 90) (layer Edge.Cuts) (width 0.15))
 (segment (start 181.864 93.036) (end 181.864 95.228974) (width 0.8128) (layer B.Cu) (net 1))
 (segment (start 181.864 95.228974) (end 183.422801 96.787775) (width 0.8128) (layer B.Cu) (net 1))
 (segment (start 183.422801 96.787775) (end 183.422801 98.284225) (width 0.8128) (layer B.Cu) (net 1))
 (segment (start 183.422801 98.284225) (end 179.599026 102.108) (width 0.8128) (layer B.Cu) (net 1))
 (segment (start 179.599026 102.108) (end 179.481238 102.108) (width 0.8128) (layer B.Cu) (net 1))
 (segment (start 179.481238 102.108) (end 178.562 102.108) (width 0.8128) (layer B.Cu) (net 1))
 (segment (start 181.864 93.036) (end 175.364 93.036) (width 0.8128) (layer B.Cu) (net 1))
 (segment (start 181.7854 84.4) (end 183.344201 85.958801) (width 0.8128) (layer B.Cu) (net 1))
 (segment (start 183.344201 85.958801) (end 183.344201 91.555799) (width 0.8128) (layer B.Cu) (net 1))
 (segment (start 183.344201 91.555799) (end 182.863999 92.036001) (width 0.8128) (layer B.Cu) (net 1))
 (segment (start 182.863999 92.036001) (end 181.864 93.036) (width 0.8128) (layer B.Cu) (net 1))
 (segment (start 175.2854 84.4) (end 181.7854 84.4) (width 0.8128) (layer B.Cu) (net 1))
 (segment (start 175.26 78.24089) (end 175.2854 78.26629) (width 0.8128) (layer B.Cu) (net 1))
 (segment (start 175.2854 78.26629) (end 175.2854 84.4) (width 0.8128) (layer B.Cu) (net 1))
 (segment (start 144.322801 82.397599) (end 142.62 82.397599) (width 0.8128) (layer B.Cu) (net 1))
 (segment (start 142.62 82.397599) (end 139.62 82.397599) (width 0.8128) (layer B.Cu) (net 1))
 (segment (start 142.24 83.82) (end 142.24 82.777599) (width 0.8128) (layer B.Cu) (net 1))
 (segment (start 142.24 82.777599) (end 142.62 82.397599) (width 0.8128) (layer B.Cu) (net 1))
 (segment (start 139.7 82.477599) (end 139.62 82.397599) (width 0.8128) (layer B.Cu) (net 1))
 (segment (start 139.62 82.397599) (end 138.236959 82.397599) (width 0.8128) (layer B.Cu) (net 1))
 (segment (start 139.7 83.82) (end 139.7 82.477599) (width 0.8128) (layer B.Cu) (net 1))
 (segment (start 146.812 79.756) (end 146.812 79.9084) (width 0.8128) (layer B.Cu) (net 1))
 (segment (start 146.812 79.9084) (end 144.322801 82.397599) (width 0.8128) (layer B.Cu) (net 1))
 (segment (start 138.236959 82.397599) (end 137.16 83.474558) (width 0.8128) (layer B.Cu) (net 1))
 (segment (start 137.16 83.474558) (end 137.16 83.82) (width 0.8128) (layer B.Cu) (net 1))
 (segment (start 180.34 73.66) (end 179.84089 73.66) (width 0.8128) (layer B.Cu) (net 1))
 (segment (start 179.84089 73.66) (end 175.26 78.24089) (width 0.8128) (layer B.Cu) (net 1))
 (segment (start 156.718 79.756) (end 156.718 104.2924) (width 0.8128) (layer B.Cu) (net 1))
 (segment (start 156.718 104.2924) (end 159.6136 107.188) (width 0.8128) (layer B.Cu) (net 1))
 (segment (start 159.6136 107.188) (end 161.29 107.188) (width 0.8128) (layer B.Cu) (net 1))
 (segment (start 146.812 75.184) (end 146.812 75.0316) (width 0.8128) (layer B.Cu) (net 1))
 (segment (start 145.1356 73.3552) (end 140.3096 73.3552) (width 0.8128) (layer B.Cu) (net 1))
 (segment (start 146.812 75.0316) (end 145.1356 73.3552) (width 0.8128) (layer B.Cu) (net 1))
 (segment (start 140.3096 73.3552) (end 138.9888 74.676) (width 0.8128) (layer B.Cu) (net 1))
 (segment (start 138.9888 74.676) (end 137.16 74.676) (width 0.8128) (layer B.Cu) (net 1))
 (segment (start 146.812 75.184) (end 146.812 79.756) (width 0.8128) (layer B.Cu) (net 1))
 (segment (start 156.718 75.184) (end 156.718 75.0316) (width 0.8128) (layer B.Cu) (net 1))
 (segment (start 155.0416 73.3552) (end 150.3172 73.3552) (width 0.8128) (layer B.Cu) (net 1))
 (segment (start 156.718 75.0316) (end 155.0416 73.3552) (width 0.8128) (layer B.Cu) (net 1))
 (segment (start 150.3172 73.3552) (end 148.4884 75.184) (width 0.8128) (layer B.Cu) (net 1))
 (segment (start 148.4884 75.184) (end 146.812 75.184) (width 0.8128) (layer B.Cu) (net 1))
 (segment (start 156.718 75.184) (end 156.718 79.756) (width 0.8128) (layer B.Cu) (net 1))
 (segment (start 155.956 68.58) (end 155.956 74.422) (width 0.8128) (layer B.Cu) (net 1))
 (segment (start 155.956 74.422) (end 156.718 75.184) (width 0.8128) (layer B.Cu) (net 1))
 (segment (start 173.228 68.58) (end 171.399199 66.751199) (width 0.8128) (layer B.Cu) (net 1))
 (segment (start 171.399199 66.751199) (end 163.139073 66.751199) (width 0.8128) (layer B.Cu) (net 1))
 (segment (start 163.139073 66.751199) (end 161.310272 68.58) (width 0.8128) (layer B.Cu) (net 1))
 (segment (start 161.310272 68.58) (end 157.752051 68.58) (width 0.8128) (layer B.Cu) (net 1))
 (segment (start 157.752051 68.58) (end 155.956 68.58) (width 0.8128) (layer B.Cu) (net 1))
 (segment (start 172.212 75.692) (end 174.244 73.66) (width 0.8128) (layer B.Cu) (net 1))
 (segment (start 174.244 73.66) (end 180.34 73.66) (width 0.8128) (layer B.Cu) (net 1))
 (segment (start 173.228 68.58) (end 173.228 74.676) (width 0.8128) (layer B.Cu) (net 1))
 (segment (start 173.228 74.676) (end 172.212 75.692) (width 0.8128) (layer B.Cu) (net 1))
 (segment (start 137.16 77.216) (end 135.89 77.216) (width 0.254) (layer F.Cu) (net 2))
 (segment (start 135.89 77.216) (end 135.86459 77.24141) (width 0.254) (layer F.Cu) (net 2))
 (segment (start 135.86459 77.24141) (end 135.86459 110.326104) (width 0.254) (layer F.Cu) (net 2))
 (segment (start 135.86459 110.326104) (end 138.441496 112.90301) (width 0.254) (layer F.Cu) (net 2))
 (segment (start 138.441496 112.90301) (end 158.11499 112.90301) (width 0.254) (layer F.Cu) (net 2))
 (segment (start 158.11499 112.90301) (end 160.426401 110.591599) (width 0.254) (layer F.Cu) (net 2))
 (segment (start 160.426401 110.591599) (end 161.29 109.728) (width 0.254) (layer F.Cu) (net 2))
 (segment (start 137.16 79.756) (end 138.43 79.756) (width 0.254) (layer F.Cu) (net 5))
 (segment (start 163.448999 108.584999) (end 167.513001 108.584999) (width 0.254) (layer F.Cu) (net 5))
 (segment (start 138.43 79.756) (end 141.350999 82.676999) (width 0.254) (layer F.Cu) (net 5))
 (segment (start 141.350999 82.676999) (end 153.639521 82.676999) (width 0.254) (layer F.Cu) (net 5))
 (segment (start 162.686999 107.822999) (end 163.448999 108.584999) (width 0.254) (layer F.Cu) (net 5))
 (segment (start 153.639521 82.676999) (end 153.695401 82.732879) (width 0.254) (layer F.Cu) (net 5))
 (segment (start 153.695401 82.732879) (end 153.695401 84.907121) (width 0.254) (layer F.Cu) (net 5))
 (segment (start 153.695401 84.907121) (end 162.686999 93.898719) (width 0.254) (layer F.Cu) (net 5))
 (segment (start 162.686999 93.898719) (end 162.686999 107.822999) (width 0.254) (layer F.Cu) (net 5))
 (segment (start 167.513001 108.584999) (end 168.046401 108.051599) (width 0.254) (layer F.Cu) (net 5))
 (segment (start 168.046401 108.051599) (end 168.91 107.188) (width 0.254) (layer F.Cu) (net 5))
 (segment (start 172.212 79.192) (end 179.888 79.192) (width 0.8128) (layer F.Cu) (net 6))
 (segment (start 179.888 79.192) (end 180.34 78.74) (width 0.8128) (layer F.Cu) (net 6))
 (segment (start 172.212 79.192) (end 172.212 77.7292) (width 0.8128) (layer F.Cu) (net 6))
 (segment (start 161.798 75.946) (end 170.4288 75.946) (width 0.8128) (layer F.Cu) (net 6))
 (segment (start 170.4288 75.946) (end 172.212 77.7292) (width 0.8128) (layer F.Cu) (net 6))
 (segment (start 154.774899 84.747101) (end 154.774899 82.054701) (width 0.254) (layer F.Cu) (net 3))
 (segment (start 154.774899 82.054701) (end 155.5496 81.28) (width 0.254) (layer F.Cu) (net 3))
 (segment (start 154.432 87.63) (end 154.774899 87.287101) (width 0.254) (layer B.Cu) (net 3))
 (segment (start 154.774899 87.287101) (end 154.774899 84.747101) (width 0.254) (layer B.Cu) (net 3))
 (segment (start 154.3304 107.442) (end 154.3304 87.7316) (width 0.254) (layer F.Cu) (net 3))
 (segment (start 154.3304 87.7316) (end 154.432 87.63) (width 0.254) (layer F.Cu) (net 3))
 (segment (start 152.5524 109.22) (end 154.3304 107.442) (width 0.254) (layer F.Cu) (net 3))
 (segment (start 152.4 109.22) (end 152.5524 109.22) (width 0.254) (layer F.Cu) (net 3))
 (segment (start 150.876 68.58) (end 149.326599 67.030599) (width 0.254) (layer F.Cu) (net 3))
 (segment (start 140.588999 70.739001) (end 140.588999 80.995521) (width 0.254) (layer F.Cu) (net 3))
 (segment (start 149.326599 67.030599) (end 144.297401 67.030599) (width 0.254) (layer F.Cu) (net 3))
 (segment (start 144.297401 67.030599) (end 140.588999 70.739001) (width 0.254) (layer F.Cu) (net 3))
 (segment (start 140.588999 80.995521) (end 140.644879 81.051401) (width 0.254) (layer F.Cu) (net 3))
 (segment (start 140.644879 81.051401) (end 143.128999 81.051401) (width 0.254) (layer F.Cu) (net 3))
 (segment (start 143.128999 81.051401) (end 144.272 79.9084) (width 0.254) (layer F.Cu) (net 3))
 (segment (start 144.272 79.9084) (end 144.272 79.756) (width 0.254) (layer F.Cu) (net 3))
 (segment (start 144.272 79.756) (end 144.272 78.486) (width 0.254) (layer F.Cu) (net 3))
 (segment (start 144.272 78.486) (end 144.272 75.184) (width 0.254) (layer F.Cu) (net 3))
 (segment (start 154.178 79.756) (end 154.178 79.9084) (width 0.254) (layer F.Cu) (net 3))
 (segment (start 153.03499 81.05141) (end 145.41501 81.05141) (width 0.254) (layer F.Cu) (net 3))
 (segment (start 154.178 79.9084) (end 153.03499 81.05141) (width 0.254) (layer F.Cu) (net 3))
 (segment (start 145.41501 81.05141) (end 144.272 79.9084) (width 0.254) (layer F.Cu) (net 3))
 (segment (start 154.178 79.756) (end 154.178 75.184) (width 0.254) (layer F.Cu) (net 3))
 (segment (start 165.74724 81.28) (end 155.5496 81.28) (width 0.254) (layer F.Cu) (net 3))
 (segment (start 155.5496 81.28) (end 154.178 79.9084) (width 0.254) (layer F.Cu) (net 3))
 (segment (start 168.656 92.456) (end 168.656 84.18876) (width 0.254) (layer F.Cu) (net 3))
 (segment (start 168.656 84.18876) (end 165.74724 81.28) (width 0.254) (layer F.Cu) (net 3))
 (segment (start 163.83 107.188) (end 163.83 97.282) (width 0.254) (layer F.Cu) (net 3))
 (segment (start 163.83 97.282) (end 168.656 92.456) (width 0.254) (layer F.Cu) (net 3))
 (segment (start 162.052 105.156) (end 162.433001 105.537001) (width 0.254) (layer B.Cu) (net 4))
 (segment (start 162.433001 105.537001) (end 162.433001 108.331001) (width 0.254) (layer B.Cu) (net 4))
 (segment (start 162.433001 108.331001) (end 162.966401 108.864401) (width 0.254) (layer B.Cu) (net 4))
 (segment (start 162.966401 108.864401) (end 163.83 109.728) (width 0.254) (layer B.Cu) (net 4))
 (segment (start 161.036 93.472) (end 162.20441 94.64041) (width 0.254) (layer F.Cu) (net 4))
 (segment (start 162.20441 94.64041) (end 162.20441 105.00359) (width 0.254) (layer F.Cu) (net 4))
 (segment (start 162.20441 105.00359) (end 162.052 105.156) (width 0.254) (layer F.Cu) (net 4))
 (segment (start 162.306 92.202) (end 161.036 93.472) (width 0.254) (layer B.Cu) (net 4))
 (segment (start 164.592 89.408) (end 162.306 91.694) (width 0.254) (layer F.Cu) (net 4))
 (segment (start 162.306 91.694) (end 162.306 92.202) (width 0.254) (layer F.Cu) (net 4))
 (via (at 154.774899 84.747101) (size 0.6858) (layers F.Cu B.Cu) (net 3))
 (via (at 154.432 87.63) (size 0.6858) (layers F.Cu B.Cu) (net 3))
 (via (at 162.052 105.156) (size 0.6858) (layers F.Cu B.Cu) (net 4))
 (via (at 161.036 93.472) (size 0.6858) (layers F.Cu B.Cu) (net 4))
 (via (at 162.306 92.202) (size 0.6858) (layers F.Cu B.Cu) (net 4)))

